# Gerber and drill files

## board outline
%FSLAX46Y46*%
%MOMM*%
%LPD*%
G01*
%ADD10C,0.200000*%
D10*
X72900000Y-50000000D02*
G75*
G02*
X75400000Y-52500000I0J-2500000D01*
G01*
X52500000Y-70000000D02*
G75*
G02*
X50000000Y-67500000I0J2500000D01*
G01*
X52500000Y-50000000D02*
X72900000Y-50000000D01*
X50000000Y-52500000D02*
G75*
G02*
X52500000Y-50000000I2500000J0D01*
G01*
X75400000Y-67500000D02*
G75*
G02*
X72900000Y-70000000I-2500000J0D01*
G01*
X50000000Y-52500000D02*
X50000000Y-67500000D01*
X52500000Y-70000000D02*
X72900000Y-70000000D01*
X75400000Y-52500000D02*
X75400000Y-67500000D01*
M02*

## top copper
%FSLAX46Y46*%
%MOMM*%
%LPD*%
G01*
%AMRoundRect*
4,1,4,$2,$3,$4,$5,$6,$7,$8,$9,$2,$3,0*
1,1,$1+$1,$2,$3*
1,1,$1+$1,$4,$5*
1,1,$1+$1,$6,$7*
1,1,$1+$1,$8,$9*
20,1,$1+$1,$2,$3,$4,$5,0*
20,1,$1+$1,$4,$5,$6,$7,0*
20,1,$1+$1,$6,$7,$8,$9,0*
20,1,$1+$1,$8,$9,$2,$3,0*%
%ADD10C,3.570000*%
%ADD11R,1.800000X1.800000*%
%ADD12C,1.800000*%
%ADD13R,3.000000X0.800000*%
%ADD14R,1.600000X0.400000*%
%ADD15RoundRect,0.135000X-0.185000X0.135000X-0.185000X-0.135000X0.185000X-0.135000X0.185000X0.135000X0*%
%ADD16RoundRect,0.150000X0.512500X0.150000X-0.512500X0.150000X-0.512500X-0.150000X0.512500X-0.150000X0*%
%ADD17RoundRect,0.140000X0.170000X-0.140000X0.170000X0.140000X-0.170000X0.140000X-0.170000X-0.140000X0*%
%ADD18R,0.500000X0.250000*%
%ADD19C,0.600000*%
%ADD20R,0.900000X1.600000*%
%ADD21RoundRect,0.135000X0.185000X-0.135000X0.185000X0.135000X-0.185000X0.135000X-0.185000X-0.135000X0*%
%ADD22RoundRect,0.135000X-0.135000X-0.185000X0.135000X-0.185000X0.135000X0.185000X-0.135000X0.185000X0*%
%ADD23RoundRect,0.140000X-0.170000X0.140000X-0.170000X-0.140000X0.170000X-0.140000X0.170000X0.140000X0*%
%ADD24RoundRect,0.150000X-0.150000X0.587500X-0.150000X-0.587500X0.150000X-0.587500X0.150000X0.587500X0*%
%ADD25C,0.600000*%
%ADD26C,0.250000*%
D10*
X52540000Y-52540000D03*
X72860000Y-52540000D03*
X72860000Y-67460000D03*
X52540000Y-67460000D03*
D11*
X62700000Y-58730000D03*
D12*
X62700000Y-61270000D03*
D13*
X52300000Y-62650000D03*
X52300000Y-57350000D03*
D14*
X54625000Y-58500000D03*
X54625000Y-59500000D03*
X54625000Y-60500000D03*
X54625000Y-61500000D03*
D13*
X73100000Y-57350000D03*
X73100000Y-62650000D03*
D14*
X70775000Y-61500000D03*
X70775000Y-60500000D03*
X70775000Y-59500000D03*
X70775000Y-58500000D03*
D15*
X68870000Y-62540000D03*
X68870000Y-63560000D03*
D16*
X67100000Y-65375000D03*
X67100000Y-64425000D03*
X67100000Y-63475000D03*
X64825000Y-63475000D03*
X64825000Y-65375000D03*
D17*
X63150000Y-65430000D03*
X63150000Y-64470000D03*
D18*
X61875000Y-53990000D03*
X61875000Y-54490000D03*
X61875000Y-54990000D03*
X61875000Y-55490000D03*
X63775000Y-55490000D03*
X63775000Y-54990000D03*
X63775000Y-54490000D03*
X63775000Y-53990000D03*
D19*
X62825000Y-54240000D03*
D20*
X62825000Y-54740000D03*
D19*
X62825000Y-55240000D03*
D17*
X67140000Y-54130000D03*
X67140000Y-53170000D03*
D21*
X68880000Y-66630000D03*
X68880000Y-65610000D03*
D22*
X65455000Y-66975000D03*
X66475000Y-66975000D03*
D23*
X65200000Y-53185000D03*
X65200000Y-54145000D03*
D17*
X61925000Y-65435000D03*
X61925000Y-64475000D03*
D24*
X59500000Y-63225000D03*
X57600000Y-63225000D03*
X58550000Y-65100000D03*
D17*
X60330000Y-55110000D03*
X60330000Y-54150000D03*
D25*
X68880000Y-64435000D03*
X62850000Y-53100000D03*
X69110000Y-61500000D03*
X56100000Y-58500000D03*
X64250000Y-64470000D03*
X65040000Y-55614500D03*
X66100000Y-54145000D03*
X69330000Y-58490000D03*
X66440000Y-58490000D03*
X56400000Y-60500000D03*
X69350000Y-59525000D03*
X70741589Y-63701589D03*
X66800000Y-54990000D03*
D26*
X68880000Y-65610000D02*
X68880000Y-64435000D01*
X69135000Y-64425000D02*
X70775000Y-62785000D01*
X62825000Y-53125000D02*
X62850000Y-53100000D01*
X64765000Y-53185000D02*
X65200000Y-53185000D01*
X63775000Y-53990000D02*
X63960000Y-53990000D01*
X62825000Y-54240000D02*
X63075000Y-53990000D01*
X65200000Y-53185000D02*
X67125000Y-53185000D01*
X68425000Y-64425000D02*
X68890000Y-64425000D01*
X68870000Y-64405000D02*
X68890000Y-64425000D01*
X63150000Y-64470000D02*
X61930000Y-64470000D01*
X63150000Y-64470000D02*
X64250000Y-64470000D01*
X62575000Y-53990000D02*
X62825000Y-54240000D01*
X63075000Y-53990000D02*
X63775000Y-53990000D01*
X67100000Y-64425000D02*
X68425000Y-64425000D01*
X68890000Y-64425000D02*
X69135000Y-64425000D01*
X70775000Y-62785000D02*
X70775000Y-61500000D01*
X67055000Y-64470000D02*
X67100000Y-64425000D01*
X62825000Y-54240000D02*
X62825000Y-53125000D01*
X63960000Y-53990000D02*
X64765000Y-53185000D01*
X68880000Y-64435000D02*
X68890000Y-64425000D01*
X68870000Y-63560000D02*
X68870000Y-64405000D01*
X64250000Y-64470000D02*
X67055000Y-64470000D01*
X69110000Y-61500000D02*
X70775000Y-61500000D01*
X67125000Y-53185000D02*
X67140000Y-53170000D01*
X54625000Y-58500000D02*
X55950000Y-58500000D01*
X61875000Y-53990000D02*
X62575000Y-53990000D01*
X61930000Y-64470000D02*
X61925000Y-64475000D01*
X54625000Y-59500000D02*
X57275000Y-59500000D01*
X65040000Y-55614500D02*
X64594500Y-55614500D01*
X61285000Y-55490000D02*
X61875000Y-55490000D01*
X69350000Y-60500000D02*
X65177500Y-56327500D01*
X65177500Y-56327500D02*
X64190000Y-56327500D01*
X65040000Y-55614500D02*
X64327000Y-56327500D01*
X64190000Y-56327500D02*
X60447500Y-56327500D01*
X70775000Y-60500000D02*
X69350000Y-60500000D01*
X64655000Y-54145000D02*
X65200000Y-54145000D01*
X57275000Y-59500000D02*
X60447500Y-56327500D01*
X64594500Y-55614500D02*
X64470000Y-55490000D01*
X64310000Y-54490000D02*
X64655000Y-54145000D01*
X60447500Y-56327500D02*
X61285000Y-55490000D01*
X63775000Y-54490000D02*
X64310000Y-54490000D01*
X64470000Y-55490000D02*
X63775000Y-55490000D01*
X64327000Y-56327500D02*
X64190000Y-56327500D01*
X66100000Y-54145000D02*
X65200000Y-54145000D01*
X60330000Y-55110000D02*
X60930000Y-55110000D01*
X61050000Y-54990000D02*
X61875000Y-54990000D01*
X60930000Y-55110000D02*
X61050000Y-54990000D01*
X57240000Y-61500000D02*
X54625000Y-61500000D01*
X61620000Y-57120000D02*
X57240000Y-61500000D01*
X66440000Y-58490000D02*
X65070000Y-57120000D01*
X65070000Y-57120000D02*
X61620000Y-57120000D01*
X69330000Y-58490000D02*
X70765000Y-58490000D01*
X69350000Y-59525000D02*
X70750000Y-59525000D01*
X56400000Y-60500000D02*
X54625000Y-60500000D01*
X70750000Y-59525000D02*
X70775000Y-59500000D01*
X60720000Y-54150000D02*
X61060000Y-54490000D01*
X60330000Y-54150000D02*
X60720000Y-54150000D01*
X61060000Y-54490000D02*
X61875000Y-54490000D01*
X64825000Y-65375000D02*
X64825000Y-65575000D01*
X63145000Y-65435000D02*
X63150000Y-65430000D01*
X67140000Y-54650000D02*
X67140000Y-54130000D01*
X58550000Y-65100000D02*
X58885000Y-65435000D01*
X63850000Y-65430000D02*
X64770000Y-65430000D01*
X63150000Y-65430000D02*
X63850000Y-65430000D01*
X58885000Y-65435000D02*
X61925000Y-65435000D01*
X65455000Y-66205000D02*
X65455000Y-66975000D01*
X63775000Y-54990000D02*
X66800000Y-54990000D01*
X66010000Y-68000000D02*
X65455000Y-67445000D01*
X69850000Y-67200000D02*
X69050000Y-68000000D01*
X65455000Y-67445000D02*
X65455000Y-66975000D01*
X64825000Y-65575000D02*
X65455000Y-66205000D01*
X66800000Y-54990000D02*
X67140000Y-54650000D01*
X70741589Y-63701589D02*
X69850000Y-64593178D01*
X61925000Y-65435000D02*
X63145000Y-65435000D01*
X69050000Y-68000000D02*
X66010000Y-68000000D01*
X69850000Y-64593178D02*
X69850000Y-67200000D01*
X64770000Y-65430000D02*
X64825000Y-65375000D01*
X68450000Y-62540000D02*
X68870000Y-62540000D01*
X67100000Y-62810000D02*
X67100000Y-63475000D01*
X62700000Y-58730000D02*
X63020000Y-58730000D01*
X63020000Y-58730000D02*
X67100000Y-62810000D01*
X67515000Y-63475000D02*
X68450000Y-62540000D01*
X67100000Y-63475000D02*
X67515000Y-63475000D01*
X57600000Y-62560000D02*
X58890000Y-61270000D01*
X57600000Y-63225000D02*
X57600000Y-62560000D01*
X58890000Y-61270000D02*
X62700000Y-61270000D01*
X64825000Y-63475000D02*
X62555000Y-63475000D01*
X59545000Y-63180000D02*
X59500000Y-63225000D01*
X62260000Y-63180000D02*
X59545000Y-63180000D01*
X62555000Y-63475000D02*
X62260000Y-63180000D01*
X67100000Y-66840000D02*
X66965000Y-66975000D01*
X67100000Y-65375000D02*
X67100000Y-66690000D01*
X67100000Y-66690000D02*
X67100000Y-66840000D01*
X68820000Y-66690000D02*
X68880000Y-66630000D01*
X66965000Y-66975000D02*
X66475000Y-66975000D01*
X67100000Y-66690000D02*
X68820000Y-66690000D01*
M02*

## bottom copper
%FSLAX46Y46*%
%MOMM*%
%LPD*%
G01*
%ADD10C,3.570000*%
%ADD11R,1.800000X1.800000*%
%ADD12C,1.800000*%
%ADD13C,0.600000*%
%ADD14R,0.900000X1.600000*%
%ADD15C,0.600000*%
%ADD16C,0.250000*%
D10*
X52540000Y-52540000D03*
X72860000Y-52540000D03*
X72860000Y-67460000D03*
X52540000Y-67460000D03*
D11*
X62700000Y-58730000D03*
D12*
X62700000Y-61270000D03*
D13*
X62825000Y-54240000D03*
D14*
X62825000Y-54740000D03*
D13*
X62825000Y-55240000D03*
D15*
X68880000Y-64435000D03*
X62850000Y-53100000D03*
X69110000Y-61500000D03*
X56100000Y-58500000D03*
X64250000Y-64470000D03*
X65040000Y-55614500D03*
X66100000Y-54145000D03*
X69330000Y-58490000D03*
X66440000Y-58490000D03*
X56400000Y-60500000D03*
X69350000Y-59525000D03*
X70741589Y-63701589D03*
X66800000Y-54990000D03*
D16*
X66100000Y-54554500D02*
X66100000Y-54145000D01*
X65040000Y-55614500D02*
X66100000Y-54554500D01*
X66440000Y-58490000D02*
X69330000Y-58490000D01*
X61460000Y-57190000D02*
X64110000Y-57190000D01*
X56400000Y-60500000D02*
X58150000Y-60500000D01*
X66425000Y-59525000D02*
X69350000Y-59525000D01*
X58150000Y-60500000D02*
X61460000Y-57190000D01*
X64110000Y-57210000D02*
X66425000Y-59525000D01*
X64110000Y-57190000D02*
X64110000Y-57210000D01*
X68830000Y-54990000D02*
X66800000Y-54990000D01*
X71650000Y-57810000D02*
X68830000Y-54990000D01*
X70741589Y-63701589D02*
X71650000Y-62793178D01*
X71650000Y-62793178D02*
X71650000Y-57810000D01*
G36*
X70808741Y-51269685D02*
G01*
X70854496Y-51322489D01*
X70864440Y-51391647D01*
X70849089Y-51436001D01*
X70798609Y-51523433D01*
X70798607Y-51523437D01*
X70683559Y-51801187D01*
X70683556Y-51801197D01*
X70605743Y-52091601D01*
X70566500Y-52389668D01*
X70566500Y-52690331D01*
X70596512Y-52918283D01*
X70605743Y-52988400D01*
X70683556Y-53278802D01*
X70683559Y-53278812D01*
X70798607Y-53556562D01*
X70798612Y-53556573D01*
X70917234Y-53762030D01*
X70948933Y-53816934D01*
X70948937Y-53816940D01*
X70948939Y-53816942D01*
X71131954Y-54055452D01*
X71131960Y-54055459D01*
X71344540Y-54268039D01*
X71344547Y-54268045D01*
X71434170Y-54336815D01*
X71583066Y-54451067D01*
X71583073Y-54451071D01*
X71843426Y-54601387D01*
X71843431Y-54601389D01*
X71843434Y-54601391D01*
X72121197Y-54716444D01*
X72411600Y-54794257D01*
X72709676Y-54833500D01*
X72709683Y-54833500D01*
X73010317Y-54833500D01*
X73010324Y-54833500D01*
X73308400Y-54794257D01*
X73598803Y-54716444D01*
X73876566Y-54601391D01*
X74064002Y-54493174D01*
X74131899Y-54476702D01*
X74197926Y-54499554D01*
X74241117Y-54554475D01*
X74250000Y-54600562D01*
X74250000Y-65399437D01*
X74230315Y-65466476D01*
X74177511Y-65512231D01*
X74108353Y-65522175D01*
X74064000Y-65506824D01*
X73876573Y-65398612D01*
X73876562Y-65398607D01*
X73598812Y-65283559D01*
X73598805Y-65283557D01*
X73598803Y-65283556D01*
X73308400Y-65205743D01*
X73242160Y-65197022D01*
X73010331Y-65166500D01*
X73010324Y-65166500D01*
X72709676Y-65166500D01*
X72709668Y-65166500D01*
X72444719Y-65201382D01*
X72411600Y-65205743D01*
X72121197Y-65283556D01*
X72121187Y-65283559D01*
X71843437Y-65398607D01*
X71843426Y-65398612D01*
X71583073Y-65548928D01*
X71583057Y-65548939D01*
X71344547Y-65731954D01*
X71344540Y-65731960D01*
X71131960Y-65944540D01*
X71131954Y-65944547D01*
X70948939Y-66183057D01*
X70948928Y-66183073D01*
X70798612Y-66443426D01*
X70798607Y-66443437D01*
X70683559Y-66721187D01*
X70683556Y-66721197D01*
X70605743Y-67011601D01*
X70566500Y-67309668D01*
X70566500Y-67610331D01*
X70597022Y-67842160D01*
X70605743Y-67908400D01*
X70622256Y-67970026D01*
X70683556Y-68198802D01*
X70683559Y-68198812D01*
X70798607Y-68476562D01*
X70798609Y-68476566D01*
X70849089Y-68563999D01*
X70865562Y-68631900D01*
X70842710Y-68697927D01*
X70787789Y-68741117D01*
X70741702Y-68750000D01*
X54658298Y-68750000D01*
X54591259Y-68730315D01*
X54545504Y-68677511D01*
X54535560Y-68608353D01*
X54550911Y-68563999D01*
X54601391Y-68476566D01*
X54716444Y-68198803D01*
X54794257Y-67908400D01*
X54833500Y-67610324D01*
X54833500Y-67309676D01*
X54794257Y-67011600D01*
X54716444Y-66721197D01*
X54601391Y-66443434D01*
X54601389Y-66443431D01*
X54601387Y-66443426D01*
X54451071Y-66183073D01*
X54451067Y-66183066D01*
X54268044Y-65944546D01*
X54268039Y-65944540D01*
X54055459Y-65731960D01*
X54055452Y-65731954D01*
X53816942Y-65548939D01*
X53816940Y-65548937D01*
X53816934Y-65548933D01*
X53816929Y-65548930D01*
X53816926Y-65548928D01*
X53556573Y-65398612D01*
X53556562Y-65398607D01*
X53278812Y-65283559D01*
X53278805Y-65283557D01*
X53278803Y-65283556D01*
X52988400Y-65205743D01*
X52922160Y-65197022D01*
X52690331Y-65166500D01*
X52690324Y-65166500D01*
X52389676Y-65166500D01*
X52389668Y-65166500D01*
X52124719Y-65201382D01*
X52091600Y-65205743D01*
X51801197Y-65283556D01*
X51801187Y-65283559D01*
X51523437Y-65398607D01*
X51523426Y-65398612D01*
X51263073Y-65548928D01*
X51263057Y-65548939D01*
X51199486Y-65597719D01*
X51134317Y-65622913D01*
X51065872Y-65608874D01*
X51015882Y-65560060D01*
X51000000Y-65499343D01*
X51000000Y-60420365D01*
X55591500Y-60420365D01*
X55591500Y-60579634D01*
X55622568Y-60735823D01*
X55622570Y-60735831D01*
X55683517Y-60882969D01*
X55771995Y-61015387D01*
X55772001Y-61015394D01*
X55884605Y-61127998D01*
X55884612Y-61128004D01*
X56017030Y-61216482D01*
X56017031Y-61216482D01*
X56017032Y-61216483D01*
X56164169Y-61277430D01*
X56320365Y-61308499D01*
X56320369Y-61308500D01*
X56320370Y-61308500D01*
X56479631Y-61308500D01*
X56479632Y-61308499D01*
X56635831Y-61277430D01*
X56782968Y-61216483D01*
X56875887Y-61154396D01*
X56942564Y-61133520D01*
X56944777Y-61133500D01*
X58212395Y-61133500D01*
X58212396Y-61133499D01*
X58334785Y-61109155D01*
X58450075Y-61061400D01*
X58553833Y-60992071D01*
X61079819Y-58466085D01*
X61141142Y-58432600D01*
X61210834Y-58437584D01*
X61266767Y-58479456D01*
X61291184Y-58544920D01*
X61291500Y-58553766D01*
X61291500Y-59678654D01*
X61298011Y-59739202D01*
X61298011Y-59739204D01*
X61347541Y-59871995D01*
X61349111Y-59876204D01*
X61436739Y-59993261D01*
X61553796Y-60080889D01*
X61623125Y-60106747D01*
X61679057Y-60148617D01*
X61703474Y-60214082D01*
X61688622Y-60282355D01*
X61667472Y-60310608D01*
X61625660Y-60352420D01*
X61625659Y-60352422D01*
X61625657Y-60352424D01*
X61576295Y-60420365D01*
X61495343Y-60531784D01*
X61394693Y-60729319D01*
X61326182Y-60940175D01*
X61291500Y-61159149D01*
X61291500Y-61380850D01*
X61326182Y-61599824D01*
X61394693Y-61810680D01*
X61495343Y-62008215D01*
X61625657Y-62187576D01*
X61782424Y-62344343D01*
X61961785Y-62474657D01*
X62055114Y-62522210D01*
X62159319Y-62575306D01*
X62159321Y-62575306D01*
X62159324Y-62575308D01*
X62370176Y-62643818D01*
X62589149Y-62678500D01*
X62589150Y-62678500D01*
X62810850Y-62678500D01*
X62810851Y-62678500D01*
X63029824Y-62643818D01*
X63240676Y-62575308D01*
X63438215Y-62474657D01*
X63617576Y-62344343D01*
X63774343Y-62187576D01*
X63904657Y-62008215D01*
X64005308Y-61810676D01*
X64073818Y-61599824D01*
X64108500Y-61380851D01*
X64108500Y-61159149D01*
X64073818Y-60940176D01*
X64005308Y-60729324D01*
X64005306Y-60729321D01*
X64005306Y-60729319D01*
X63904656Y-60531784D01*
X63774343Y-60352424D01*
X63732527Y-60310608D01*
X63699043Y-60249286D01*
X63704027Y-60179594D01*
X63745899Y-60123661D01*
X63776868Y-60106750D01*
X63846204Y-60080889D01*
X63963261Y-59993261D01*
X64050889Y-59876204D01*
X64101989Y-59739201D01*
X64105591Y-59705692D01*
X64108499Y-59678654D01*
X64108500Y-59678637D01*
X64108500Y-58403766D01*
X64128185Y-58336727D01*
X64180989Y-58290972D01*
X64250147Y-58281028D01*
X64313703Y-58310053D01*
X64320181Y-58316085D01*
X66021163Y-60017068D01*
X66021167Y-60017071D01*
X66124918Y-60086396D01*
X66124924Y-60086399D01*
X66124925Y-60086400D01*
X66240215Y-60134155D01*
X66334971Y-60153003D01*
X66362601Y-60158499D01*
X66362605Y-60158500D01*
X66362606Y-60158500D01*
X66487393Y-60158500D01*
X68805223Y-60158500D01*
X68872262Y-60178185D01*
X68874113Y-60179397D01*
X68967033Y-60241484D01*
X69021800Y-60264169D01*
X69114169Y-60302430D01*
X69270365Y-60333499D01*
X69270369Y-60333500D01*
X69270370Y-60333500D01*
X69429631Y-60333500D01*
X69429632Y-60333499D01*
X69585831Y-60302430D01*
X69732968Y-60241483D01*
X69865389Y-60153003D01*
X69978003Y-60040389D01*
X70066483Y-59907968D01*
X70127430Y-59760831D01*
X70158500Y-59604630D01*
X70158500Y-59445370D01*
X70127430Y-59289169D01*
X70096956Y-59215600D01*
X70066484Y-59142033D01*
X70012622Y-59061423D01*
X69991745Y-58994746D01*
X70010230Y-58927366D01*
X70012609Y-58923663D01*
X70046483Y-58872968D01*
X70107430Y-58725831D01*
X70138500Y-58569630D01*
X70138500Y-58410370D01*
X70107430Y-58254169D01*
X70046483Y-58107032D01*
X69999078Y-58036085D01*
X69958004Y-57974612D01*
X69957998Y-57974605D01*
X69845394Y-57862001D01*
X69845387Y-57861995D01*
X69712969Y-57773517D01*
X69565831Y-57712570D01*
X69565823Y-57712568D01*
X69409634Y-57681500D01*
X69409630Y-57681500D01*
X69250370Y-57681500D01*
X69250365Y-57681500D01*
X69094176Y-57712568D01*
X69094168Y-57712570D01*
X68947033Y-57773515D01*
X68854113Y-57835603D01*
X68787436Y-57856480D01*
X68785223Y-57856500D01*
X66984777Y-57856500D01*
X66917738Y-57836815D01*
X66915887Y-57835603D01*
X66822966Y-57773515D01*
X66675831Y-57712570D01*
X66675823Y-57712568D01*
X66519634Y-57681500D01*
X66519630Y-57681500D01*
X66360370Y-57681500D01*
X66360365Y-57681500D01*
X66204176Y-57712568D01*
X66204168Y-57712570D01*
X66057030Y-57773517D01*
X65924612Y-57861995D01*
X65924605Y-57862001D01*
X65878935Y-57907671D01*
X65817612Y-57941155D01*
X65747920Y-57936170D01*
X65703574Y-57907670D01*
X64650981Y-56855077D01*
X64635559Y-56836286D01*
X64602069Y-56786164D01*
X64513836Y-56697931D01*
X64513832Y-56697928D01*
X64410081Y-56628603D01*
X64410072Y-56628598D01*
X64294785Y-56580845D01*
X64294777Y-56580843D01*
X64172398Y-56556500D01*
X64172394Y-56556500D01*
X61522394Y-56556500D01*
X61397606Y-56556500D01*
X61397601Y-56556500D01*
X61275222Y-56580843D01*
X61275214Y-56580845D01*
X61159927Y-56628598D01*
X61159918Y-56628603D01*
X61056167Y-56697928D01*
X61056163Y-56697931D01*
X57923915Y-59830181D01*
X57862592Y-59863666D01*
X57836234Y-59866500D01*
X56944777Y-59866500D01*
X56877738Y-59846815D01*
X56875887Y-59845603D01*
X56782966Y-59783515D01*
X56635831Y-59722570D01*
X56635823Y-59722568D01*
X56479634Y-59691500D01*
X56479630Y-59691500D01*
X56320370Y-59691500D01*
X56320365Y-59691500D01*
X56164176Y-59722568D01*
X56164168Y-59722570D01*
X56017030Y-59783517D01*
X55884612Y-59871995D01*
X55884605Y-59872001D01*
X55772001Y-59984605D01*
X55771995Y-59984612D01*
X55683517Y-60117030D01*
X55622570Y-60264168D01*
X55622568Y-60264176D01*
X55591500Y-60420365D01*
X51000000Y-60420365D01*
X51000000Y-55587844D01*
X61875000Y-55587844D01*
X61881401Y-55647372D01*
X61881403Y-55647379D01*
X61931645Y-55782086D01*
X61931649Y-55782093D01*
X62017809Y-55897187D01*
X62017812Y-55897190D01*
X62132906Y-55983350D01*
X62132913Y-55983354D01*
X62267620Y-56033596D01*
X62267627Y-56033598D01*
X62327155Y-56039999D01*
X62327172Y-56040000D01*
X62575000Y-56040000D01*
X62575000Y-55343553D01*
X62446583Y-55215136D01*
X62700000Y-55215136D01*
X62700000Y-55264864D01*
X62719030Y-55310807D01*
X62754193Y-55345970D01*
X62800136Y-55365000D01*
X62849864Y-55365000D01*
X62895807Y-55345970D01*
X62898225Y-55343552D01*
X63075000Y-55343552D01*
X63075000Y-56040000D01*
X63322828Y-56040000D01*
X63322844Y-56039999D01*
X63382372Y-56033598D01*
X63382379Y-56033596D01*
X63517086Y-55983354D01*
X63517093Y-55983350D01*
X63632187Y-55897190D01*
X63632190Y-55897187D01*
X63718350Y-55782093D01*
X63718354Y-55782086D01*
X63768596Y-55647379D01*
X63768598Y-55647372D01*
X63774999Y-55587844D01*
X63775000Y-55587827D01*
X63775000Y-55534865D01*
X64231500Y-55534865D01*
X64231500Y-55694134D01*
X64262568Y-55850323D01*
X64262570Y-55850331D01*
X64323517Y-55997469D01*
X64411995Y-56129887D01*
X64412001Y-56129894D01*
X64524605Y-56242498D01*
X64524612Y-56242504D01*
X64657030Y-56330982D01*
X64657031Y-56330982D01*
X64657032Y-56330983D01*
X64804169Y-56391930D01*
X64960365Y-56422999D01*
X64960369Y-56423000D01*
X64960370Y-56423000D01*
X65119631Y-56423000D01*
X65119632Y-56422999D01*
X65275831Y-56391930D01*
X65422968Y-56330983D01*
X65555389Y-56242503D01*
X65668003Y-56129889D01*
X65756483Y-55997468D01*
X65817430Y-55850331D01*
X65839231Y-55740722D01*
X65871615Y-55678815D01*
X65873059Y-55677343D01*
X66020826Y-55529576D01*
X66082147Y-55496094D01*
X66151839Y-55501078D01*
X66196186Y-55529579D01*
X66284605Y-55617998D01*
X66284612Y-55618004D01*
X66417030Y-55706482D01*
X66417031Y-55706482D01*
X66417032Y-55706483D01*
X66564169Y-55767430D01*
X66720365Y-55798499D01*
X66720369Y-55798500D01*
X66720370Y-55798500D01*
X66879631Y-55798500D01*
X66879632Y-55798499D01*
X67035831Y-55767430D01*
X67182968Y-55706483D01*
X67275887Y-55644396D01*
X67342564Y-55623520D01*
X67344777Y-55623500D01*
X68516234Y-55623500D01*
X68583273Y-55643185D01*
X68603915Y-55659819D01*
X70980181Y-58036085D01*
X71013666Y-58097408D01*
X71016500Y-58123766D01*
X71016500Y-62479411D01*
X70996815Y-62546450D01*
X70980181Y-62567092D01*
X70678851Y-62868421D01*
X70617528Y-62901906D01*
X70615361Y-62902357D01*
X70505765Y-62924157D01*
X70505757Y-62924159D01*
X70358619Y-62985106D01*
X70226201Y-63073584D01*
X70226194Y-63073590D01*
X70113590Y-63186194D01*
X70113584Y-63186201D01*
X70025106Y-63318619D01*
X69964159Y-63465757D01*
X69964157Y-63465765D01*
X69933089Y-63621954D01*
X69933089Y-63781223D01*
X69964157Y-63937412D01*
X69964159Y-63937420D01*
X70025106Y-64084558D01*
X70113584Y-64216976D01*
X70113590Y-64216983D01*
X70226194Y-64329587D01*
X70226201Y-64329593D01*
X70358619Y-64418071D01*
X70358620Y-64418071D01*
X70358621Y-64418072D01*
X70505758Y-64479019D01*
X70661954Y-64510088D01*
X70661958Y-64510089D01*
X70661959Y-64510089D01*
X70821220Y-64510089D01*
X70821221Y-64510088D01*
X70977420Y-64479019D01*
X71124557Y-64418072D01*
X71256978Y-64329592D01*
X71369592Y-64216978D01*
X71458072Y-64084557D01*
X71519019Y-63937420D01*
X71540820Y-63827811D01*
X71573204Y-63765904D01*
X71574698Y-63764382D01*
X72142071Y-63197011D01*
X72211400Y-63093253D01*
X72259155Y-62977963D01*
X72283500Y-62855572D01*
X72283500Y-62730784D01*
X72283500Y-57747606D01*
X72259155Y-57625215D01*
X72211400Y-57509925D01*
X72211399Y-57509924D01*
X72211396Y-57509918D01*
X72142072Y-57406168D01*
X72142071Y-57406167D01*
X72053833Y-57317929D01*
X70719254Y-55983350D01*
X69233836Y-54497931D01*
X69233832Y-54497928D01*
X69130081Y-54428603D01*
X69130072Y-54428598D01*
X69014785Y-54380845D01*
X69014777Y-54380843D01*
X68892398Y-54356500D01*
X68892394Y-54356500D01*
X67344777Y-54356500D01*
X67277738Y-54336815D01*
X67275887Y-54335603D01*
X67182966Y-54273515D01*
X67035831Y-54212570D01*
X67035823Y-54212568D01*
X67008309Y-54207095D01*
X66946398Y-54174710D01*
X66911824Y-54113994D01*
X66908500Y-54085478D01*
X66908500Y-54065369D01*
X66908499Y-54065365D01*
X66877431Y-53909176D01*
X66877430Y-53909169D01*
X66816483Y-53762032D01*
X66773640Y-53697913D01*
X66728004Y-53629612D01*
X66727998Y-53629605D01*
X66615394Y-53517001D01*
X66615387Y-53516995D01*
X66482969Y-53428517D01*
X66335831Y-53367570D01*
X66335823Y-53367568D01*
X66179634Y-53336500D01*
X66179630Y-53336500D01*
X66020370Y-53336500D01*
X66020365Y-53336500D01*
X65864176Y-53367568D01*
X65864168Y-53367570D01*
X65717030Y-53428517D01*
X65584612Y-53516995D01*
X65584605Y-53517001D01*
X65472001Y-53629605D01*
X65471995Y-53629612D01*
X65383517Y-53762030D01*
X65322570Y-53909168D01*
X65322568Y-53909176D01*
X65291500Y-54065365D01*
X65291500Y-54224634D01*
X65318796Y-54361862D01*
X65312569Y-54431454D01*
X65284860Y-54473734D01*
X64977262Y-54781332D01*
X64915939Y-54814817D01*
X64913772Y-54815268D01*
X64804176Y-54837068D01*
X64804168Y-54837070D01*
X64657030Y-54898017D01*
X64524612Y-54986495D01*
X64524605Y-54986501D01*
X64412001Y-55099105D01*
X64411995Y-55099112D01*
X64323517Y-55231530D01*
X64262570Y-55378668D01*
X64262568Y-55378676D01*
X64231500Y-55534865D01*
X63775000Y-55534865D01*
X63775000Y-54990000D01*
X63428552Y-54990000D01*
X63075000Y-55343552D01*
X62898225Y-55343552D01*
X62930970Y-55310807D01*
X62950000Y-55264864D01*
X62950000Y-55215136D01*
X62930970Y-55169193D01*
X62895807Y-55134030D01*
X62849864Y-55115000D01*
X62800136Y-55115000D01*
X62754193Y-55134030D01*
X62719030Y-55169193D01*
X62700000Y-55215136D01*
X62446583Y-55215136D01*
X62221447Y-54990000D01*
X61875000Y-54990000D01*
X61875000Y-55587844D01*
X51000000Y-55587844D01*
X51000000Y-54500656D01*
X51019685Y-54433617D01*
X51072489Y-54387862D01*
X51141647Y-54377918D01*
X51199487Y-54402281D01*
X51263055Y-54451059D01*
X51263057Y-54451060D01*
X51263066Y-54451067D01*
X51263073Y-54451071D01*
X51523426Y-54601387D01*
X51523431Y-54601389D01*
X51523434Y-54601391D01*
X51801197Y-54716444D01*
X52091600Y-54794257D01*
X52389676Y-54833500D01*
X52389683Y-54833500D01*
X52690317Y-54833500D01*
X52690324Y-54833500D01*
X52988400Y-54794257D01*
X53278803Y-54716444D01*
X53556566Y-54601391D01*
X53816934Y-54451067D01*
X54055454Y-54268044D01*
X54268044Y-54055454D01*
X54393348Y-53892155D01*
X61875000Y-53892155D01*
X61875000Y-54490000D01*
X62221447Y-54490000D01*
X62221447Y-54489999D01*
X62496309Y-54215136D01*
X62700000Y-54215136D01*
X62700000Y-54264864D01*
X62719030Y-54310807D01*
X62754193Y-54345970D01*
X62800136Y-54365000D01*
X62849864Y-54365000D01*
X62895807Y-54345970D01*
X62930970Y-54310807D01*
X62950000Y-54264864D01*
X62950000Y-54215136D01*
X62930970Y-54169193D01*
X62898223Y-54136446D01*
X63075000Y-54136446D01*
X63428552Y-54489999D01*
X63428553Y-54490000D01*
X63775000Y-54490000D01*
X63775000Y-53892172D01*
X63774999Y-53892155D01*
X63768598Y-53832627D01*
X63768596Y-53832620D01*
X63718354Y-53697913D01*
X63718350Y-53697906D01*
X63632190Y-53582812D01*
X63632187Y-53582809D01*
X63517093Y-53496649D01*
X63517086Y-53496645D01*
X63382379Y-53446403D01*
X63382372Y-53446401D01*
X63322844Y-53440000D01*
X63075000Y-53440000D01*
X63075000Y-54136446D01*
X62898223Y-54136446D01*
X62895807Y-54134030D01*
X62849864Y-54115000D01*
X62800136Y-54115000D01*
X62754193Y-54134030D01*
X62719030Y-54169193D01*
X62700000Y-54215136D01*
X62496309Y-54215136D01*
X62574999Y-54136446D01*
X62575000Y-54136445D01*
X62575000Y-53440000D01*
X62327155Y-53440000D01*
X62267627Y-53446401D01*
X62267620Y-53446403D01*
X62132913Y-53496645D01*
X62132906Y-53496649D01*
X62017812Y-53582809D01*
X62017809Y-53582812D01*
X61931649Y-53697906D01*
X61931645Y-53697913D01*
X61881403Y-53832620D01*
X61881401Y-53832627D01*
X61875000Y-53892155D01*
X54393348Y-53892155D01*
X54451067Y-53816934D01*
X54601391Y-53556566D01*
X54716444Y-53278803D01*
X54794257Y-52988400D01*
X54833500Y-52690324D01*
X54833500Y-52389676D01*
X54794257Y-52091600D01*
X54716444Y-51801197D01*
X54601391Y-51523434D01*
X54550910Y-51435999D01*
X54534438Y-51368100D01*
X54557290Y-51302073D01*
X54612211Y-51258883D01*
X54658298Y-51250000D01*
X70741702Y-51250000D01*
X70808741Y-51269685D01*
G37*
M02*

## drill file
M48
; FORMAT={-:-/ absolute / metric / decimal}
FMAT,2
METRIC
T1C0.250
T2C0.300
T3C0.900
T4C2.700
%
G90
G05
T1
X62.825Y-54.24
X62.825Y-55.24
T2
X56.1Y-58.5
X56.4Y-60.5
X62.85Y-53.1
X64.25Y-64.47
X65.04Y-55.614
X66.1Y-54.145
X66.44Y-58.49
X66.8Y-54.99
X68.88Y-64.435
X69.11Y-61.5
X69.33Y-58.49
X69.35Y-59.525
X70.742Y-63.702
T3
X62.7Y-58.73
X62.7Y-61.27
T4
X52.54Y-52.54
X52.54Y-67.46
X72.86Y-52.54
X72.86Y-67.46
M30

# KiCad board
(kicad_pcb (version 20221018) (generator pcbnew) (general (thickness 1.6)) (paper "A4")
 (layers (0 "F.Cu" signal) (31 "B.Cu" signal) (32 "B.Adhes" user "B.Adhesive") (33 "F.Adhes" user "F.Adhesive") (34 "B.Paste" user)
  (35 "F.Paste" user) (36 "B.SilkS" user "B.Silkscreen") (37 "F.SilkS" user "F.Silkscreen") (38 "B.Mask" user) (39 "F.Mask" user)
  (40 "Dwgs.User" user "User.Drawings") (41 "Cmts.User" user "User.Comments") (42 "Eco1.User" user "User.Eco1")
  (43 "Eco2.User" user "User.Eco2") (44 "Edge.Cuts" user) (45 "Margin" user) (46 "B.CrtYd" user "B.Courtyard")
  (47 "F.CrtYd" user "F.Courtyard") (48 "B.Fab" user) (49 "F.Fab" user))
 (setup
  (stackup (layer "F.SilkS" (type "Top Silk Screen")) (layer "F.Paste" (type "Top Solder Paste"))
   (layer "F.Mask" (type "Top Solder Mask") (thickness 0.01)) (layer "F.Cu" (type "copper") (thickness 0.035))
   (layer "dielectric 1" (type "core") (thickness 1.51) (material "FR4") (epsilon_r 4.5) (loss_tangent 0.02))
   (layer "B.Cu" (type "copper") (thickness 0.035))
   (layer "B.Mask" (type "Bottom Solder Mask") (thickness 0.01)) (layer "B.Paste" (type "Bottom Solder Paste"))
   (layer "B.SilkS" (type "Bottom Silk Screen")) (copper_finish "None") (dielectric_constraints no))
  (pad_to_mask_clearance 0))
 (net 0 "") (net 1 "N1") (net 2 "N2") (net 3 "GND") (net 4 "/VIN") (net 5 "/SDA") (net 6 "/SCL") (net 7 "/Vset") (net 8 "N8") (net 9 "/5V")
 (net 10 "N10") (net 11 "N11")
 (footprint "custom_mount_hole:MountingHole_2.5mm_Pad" (layer "F.Cu") (at 52.54 52.54)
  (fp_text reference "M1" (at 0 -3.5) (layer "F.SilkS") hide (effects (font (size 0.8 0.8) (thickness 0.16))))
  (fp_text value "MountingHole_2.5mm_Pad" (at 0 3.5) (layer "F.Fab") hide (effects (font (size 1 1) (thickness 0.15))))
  (pad "~" thru_hole circle (at 0 0) (size 3.57 3.57) (drill 2.7) (layers "*.Cu" "*.Mask")))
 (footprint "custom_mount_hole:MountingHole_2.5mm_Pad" (layer "F.Cu") (at 72.86 52.54)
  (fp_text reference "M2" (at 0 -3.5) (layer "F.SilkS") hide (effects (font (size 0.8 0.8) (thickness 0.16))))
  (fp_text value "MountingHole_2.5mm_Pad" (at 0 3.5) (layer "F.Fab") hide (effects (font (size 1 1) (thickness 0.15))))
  (pad "~" thru_hole circle (at 0 0) (size 3.57 3.57) (drill 2.7) (layers "*.Cu" "*.Mask")))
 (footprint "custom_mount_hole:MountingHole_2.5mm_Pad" (layer "F.Cu") (at 72.86 67.46)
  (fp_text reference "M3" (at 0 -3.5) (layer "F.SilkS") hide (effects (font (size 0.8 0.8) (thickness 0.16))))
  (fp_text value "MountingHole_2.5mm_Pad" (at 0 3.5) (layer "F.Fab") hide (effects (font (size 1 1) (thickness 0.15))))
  (pad "~" thru_hole circle (at 0 0) (size 3.57 3.57) (drill 2.7) (layers "*.Cu" "*.Mask")))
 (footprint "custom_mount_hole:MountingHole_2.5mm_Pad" (layer "F.Cu") (at 52.54 67.46)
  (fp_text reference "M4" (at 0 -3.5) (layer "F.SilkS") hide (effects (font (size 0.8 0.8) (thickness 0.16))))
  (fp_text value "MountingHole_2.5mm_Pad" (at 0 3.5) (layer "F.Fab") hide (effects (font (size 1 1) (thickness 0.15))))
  (pad "~" thru_hole circle (at 0 0) (size 3.57 3.57) (drill 2.7) (layers "*.Cu" "*.Mask")))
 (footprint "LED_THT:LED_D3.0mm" (layer "F.Cu") (at 62.7 58.73 -90)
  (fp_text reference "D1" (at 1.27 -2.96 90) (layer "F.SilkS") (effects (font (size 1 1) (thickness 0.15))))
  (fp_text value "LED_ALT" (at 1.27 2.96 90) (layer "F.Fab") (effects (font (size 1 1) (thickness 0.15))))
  (pad "1" thru_hole rect (at 0 0 270) (size 1.8 1.8) (drill 0.9) (layers "*.Cu" "*.Mask") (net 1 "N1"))
  (pad "2" thru_hole circle (at 2.54 0 270) (size 1.8 1.8) (drill 0.9) (layers "*.Cu" "*.Mask") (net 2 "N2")))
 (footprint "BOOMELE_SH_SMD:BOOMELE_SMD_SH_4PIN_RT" (layer "F.Cu") (at 52.78 60 90)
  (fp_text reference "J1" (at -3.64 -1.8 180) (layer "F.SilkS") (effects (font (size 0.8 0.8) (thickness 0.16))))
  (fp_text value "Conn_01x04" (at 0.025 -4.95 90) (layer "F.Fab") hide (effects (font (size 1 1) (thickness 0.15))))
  (pad "" smd rect (at -2.65 -0.48 270) (size 0.8 3) (layers "F.Cu" "F.Paste" "F.Mask"))
  (pad "" smd rect (at 2.65 -0.48 270) (size 0.8 3) (layers "F.Cu" "F.Paste" "F.Mask"))
  (pad "1" smd rect (at 1.5 1.845 270) (size 0.4 1.6) (layers "F.Cu" "F.Paste" "F.Mask") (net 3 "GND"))
  (pad "2" smd rect (at 0.5 1.845 270) (size 0.4 1.6) (layers "F.Cu" "F.Paste" "F.Mask") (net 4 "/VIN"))
  (pad "3" smd rect (at -0.5 1.845 270) (size 0.4 1.6) (layers "F.Cu" "F.Paste" "F.Mask") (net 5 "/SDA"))
  (pad "4" smd rect (at -1.5 1.845 270) (size 0.4 1.6) (layers "F.Cu" "F.Paste" "F.Mask") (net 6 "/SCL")))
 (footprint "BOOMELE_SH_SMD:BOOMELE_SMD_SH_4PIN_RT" (layer "F.Cu") (at 72.62 60 -90)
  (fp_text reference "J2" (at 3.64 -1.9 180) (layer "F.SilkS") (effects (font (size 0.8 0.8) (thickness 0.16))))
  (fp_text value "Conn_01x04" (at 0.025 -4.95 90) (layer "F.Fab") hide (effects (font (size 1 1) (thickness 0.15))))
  (pad "" smd rect (at -2.65 -0.48 90) (size 0.8 3) (layers "F.Cu" "F.Paste" "F.Mask"))
  (pad "" smd rect (at 2.65 -0.48 90) (size 0.8 3) (layers "F.Cu" "F.Paste" "F.Mask"))
  (pad "1" smd rect (at 1.5 1.845 90) (size 0.4 1.6) (layers "F.Cu" "F.Paste" "F.Mask") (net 3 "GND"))
  (pad "2" smd rect (at 0.5 1.845 90) (size 0.4 1.6) (layers "F.Cu" "F.Paste" "F.Mask") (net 4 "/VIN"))
  (pad "3" smd rect (at -0.5 1.845 90) (size 0.4 1.6) (layers "F.Cu" "F.Paste" "F.Mask") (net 5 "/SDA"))
  (pad "4" smd rect (at -1.5 1.845 90) (size 0.4 1.6) (layers "F.Cu" "F.Paste" "F.Mask") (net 6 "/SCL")))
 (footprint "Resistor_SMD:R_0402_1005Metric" (layer "F.Cu") (at 68.87 63.05 -90)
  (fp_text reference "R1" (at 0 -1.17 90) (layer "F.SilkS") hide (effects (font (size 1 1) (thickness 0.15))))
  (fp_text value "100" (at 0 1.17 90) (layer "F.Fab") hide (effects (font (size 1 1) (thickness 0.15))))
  (pad "1" smd roundrect (at -0.51 0 270) (size 0.54 0.64) (layers "F.Cu" "F.Paste" "F.Mask") (roundrect_rratio 0.25) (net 1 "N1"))
  (pad "2" smd roundrect (at 0.51 0 270) (size 0.54 0.64) (layers "F.Cu" "F.Paste" "F.Mask") (roundrect_rratio 0.25) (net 3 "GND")))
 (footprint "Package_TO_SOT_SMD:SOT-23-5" (layer "F.Cu") (at 65.9625 64.425 180)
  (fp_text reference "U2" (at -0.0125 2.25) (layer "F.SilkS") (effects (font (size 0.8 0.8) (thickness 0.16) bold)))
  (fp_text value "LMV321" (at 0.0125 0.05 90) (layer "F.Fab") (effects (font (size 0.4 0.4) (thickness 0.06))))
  (pad "1" smd roundrect (at -1.1375 -0.95 180) (size 1.325 0.6) (layers "F.Cu" "F.Paste" "F.Mask") (roundrect_rratio 0.25) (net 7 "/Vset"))
  (pad "2" smd roundrect (at -1.1375 0 180) (size 1.325 0.6) (layers "F.Cu" "F.Paste" "F.Mask") (roundrect_rratio 0.25) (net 3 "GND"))
  (pad "3" smd roundrect (at -1.1375 0.95 180) (size 1.325 0.6) (layers "F.Cu" "F.Paste" "F.Mask") (roundrect_rratio 0.25) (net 1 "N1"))
  (pad "4" smd roundrect (at 1.1375 0.95 180) (size 1.325 0.6) (layers "F.Cu" "F.Paste" "F.Mask") (roundrect_rratio 0.25) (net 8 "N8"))
  (pad "5" smd roundrect (at 1.1375 -0.95 180) (size 1.325 0.6) (layers "F.Cu" "F.Paste" "F.Mask") (roundrect_rratio 0.25) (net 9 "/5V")))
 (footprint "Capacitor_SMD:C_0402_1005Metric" (layer "F.Cu") (at 63.15 64.95 90)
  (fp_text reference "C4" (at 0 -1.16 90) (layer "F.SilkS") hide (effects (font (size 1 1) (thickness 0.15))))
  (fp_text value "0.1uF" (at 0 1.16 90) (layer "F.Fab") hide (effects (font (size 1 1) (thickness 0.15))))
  (pad "1" smd roundrect (at -0.48 0 90) (size 0.56 0.62) (layers "F.Cu" "F.Paste" "F.Mask") (roundrect_rratio 0.25) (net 9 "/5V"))
  (pad "2" smd roundrect (at 0.48 0 90) (size 0.56 0.62) (layers "F.Cu" "F.Paste" "F.Mask") (roundrect_rratio 0.25) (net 3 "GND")))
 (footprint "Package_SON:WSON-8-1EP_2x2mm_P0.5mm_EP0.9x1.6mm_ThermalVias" (layer "F.Cu") (at 62.825 54.74)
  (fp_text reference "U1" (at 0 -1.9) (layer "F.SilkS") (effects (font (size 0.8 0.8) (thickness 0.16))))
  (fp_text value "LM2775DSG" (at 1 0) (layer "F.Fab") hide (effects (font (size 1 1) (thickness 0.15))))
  (pad "" smd rect (at 0 -0.4) (size 0.75 0.65) (layers "F.Paste"))
  (pad "" smd rect (at 0 0.4) (size 0.75 0.65) (layers "F.Paste"))
  (pad "1" smd rect (at -0.95 -0.75) (size 0.5 0.25) (layers "F.Cu" "F.Paste" "F.Mask") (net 3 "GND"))
  (pad "2" smd rect (at -0.95 -0.25) (size 0.5 0.25) (layers "F.Cu" "F.Paste" "F.Mask") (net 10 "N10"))
  (pad "3" smd rect (at -0.95 0.25) (size 0.5 0.25) (layers "F.Cu" "F.Paste" "F.Mask") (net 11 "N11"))
  (pad "4" smd rect (at -0.95 0.75) (size 0.5 0.25) (layers "F.Cu" "F.Paste" "F.Mask") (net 4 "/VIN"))
  (pad "5" smd rect (at 0.95 0.75) (size 0.5 0.25) (layers "F.Cu" "F.Paste" "F.Mask") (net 4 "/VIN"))
  (pad "6" smd rect (at 0.95 0.25) (size 0.5 0.25) (layers "F.Cu" "F.Paste" "F.Mask") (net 9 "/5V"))
  (pad "7" smd rect (at 0.95 -0.25) (size 0.5 0.25) (layers "F.Cu" "F.Paste" "F.Mask") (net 4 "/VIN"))
  (pad "8" smd rect (at 0.95 -0.75) (size 0.5 0.25) (layers "F.Cu" "F.Paste" "F.Mask") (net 3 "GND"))
  (pad "9" thru_hole circle (at 0 -0.5) (size 0.6 0.6) (drill 0.25) (layers "*.Cu") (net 3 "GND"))
  (pad "9" smd rect (at 0 0) (size 0.9 1.6) (layers "F.Cu" "F.Mask") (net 3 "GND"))
  (pad "9" smd rect (at 0 0) (size 0.9 1.6) (layers "B.Cu") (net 3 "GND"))
  (pad "9" thru_hole circle (at 0 0.5) (size 0.6 0.6) (drill 0.25) (layers "*.Cu") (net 3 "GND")))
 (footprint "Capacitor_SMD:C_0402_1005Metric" (layer "F.Cu") (at 67.14 53.65 90)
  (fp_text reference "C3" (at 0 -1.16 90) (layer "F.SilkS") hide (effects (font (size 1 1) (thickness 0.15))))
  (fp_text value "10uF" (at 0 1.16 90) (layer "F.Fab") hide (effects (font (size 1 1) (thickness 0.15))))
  (pad "1" smd roundrect (at -0.48 0 90) (size 0.56 0.62) (layers "F.Cu" "F.Paste" "F.Mask") (roundrect_rratio 0.25) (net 9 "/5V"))
  (pad "2" smd roundrect (at 0.48 0 90) (size 0.56 0.62) (layers "F.Cu" "F.Paste" "F.Mask") (roundrect_rratio 0.25) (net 3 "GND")))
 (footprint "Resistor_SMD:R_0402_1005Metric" (layer "F.Cu") (at 68.88 66.12 90)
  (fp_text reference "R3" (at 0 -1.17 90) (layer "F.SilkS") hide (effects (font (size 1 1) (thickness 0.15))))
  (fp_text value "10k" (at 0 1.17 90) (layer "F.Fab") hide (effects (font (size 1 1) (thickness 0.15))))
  (pad "1" smd roundrect (at -0.51 0 90) (size 0.54 0.64) (layers "F.Cu" "F.Paste" "F.Mask") (roundrect_rratio 0.25) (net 7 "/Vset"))
  (pad "2" smd roundrect (at 0.51 0 90) (size 0.54 0.64) (layers "F.Cu" "F.Paste" "F.Mask") (roundrect_rratio 0.25) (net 3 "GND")))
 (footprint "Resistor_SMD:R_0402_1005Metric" (layer "F.Cu") (at 65.965 66.975)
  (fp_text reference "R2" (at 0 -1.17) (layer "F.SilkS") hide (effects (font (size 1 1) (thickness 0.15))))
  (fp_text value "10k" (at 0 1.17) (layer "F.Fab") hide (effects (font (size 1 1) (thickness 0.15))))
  (pad "1" smd roundrect (at -0.51 0) (size 0.54 0.64) (layers "F.Cu" "F.Paste" "F.Mask") (roundrect_rratio 0.25) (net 9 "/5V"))
  (pad "2" smd roundrect (at 0.51 0) (size 0.54 0.64) (layers "F.Cu" "F.Paste" "F.Mask") (roundrect_rratio 0.25) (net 7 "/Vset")))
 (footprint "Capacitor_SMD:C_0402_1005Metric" (layer "F.Cu") (at 65.2 53.665 -90)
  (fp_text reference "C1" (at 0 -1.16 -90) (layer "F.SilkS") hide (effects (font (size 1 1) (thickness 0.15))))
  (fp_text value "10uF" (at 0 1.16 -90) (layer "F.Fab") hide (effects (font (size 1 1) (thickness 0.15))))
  (pad "1" smd roundrect (at -0.48 0 270) (size 0.56 0.62) (layers "F.Cu" "F.Paste" "F.Mask") (roundrect_rratio 0.25) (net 3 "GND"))
  (pad "2" smd roundrect (at 0.48 0 270) (size 0.56 0.62) (layers "F.Cu" "F.Paste" "F.Mask") (roundrect_rratio 0.25) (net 4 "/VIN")))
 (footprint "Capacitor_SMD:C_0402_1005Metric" (layer "F.Cu") (at 61.925 64.955 90)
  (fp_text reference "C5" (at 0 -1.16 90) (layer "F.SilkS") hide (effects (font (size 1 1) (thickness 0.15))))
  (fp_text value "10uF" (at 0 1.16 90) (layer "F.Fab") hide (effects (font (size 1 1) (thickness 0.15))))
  (pad "1" smd roundrect (at -0.48 0 90) (size 0.56 0.62) (layers "F.Cu" "F.Paste" "F.Mask") (roundrect_rratio 0.25) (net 9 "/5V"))
  (pad "2" smd roundrect (at 0.48 0 90) (size 0.56 0.62) (layers "F.Cu" "F.Paste" "F.Mask") (roundrect_rratio 0.25) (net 3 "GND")))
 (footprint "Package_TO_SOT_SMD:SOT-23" (layer "F.Cu") (at 58.55 64.1625 -90)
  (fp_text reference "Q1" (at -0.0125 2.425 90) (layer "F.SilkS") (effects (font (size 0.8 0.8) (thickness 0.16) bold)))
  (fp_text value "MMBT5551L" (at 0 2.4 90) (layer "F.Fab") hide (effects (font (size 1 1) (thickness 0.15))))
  (pad "1" smd roundrect (at -0.9375 -0.95 270) (size 1.475 0.6) (layers "F.Cu" "F.Paste" "F.Mask") (roundrect_rratio 0.25) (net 8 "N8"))
  (pad "2" smd roundrect (at -0.9375 0.95 270) (size 1.475 0.6) (layers "F.Cu" "F.Paste" "F.Mask") (roundrect_rratio 0.25) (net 2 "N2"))
  (pad "3" smd roundrect (at 0.9375 0 270) (size 1.475 0.6) (layers "F.Cu" "F.Paste" "F.Mask") (roundrect_rratio 0.25) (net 9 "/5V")))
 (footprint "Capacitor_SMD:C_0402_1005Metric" (layer "F.Cu") (at 60.33 54.63 90)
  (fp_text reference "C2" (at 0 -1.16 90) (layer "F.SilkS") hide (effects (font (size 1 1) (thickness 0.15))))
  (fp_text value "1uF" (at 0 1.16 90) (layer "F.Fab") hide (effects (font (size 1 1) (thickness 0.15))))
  (pad "1" smd roundrect (at -0.48 0 90) (size 0.56 0.62) (layers "F.Cu" "F.Paste" "F.Mask") (roundrect_rratio 0.25) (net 11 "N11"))
  (pad "2" smd roundrect (at 0.48 0 90) (size 0.56 0.62) (layers "F.Cu" "F.Paste" "F.Mask") (roundrect_rratio 0.25) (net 10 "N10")))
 (gr_arc (start 72.9 50) (mid 74.667767 50.732233) (end 75.4 52.5) (stroke (width 0.2) (type solid)) (layer "Edge.Cuts"))
 (gr_arc (start 52.5 70) (mid 50.732233 69.267767) (end 50 67.5) (stroke (width 0.2) (type solid)) (layer "Edge.Cuts"))
 (gr_line (start 52.5 50) (end 72.9 50) (stroke (width 0.2) (type solid)) (layer "Edge.Cuts"))
 (gr_arc (start 50 52.5) (mid 50.732233 50.732233) (end 52.5 50) (stroke (width 0.2) (type solid)) (layer "Edge.Cuts"))
 (gr_arc (start 75.4 67.5) (mid 74.667767 69.267767) (end 72.9 70) (stroke (width 0.2) (type solid)) (layer "Edge.Cuts"))
 (gr_line (start 50 52.5) (end 50 67.5) (stroke (width 0.2) (type solid)) (layer "Edge.Cuts"))
 (gr_line (start 52.5 70) (end 72.9 70) (stroke (width 0.2) (type solid)) (layer "Edge.Cuts"))
 (gr_line (start 75.4 52.5) (end 75.4 67.5) (stroke (width 0.2) (type solid)) (layer "Edge.Cuts"))
 (segment (start 68.88 65.61) (end 68.88 64.435) (width 0.25) (layer "F.Cu") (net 3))
 (segment (start 69.135 64.425) (end 70.775 62.785) (width 0.25) (layer "F.Cu") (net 3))
 (segment (start 62.825 53.125) (end 62.85 53.1) (width 0.25) (layer "F.Cu") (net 3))
 (segment (start 64.765 53.185) (end 65.2 53.185) (width 0.25) (layer "F.Cu") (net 3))
 (segment (start 63.775 53.99) (end 63.96 53.99) (width 0.25) (layer "F.Cu") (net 3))
 (segment (start 62.825 54.24) (end 63.075 53.99) (width 0.25) (layer "F.Cu") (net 3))
 (segment (start 65.2 53.185) (end 67.125 53.185) (width 0.25) (layer "F.Cu") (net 3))
 (segment (start 68.425 64.425) (end 68.89 64.425) (width 0.25) (layer "F.Cu") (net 3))
 (segment (start 68.87 64.405) (end 68.89 64.425) (width 0.25) (layer "F.Cu") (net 3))
 (segment (start 63.15 64.47) (end 61.93 64.47) (width 0.25) (layer "F.Cu") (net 3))
 (segment (start 63.15 64.47) (end 64.25 64.47) (width 0.25) (layer "F.Cu") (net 3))
 (segment (start 62.575 53.99) (end 62.825 54.24) (width 0.25) (layer "F.Cu") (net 3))
 (segment (start 63.075 53.99) (end 63.775 53.99) (width 0.25) (layer "F.Cu") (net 3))
 (segment (start 67.1 64.425) (end 68.425 64.425) (width 0.25) (layer "F.Cu") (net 3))
 (segment (start 68.89 64.425) (end 69.135 64.425) (width 0.25) (layer "F.Cu") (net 3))
 (segment (start 70.775 62.785) (end 70.775 61.5) (width 0.25) (layer "F.Cu") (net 3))
 (segment (start 67.055 64.47) (end 67.1 64.425) (width 0.25) (layer "F.Cu") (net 3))
 (segment (start 62.825 54.24) (end 62.825 53.125) (width 0.25) (layer "F.Cu") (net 3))
 (segment (start 63.96 53.99) (end 64.765 53.185) (width 0.25) (layer "F.Cu") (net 3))
 (segment (start 68.88 64.435) (end 68.89 64.425) (width 0.25) (layer "F.Cu") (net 3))
 (segment (start 68.87 63.56) (end 68.87 64.405) (width 0.25) (layer "F.Cu") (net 3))
 (segment (start 64.25 64.47) (end 67.055 64.47) (width 0.25) (layer "F.Cu") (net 3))
 (segment (start 69.11 61.5) (end 70.775 61.5) (width 0.25) (layer "F.Cu") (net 3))
 (segment (start 67.125 53.185) (end 67.14 53.17) (width 0.25) (layer "F.Cu") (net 3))
 (segment (start 54.625 58.5) (end 55.95 58.5) (width 0.25) (layer "F.Cu") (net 3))
 (segment (start 61.875 53.99) (end 62.575 53.99) (width 0.25) (layer "F.Cu") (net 3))
 (segment (start 61.93 64.47) (end 61.925 64.475) (width 0.25) (layer "F.Cu") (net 3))
 (via (at 68.88 64.435) (size 0.6) (drill 0.3) (layers "F.Cu" "B.Cu") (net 3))
 (via (at 62.85 53.1) (size 0.6) (drill 0.3) (layers "F.Cu" "B.Cu") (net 3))
 (via (at 69.11 61.5) (size 0.6) (drill 0.3) (layers "F.Cu" "B.Cu") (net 3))
 (via (at 56.1 58.5) (size 0.6) (drill 0.3) (layers "F.Cu" "B.Cu") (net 3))
 (via (at 64.25 64.47) (size 0.6) (drill 0.3) (layers "F.Cu" "B.Cu") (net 3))
 (segment (start 54.625 59.5) (end 57.275 59.5) (width 0.25) (layer "F.Cu") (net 4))
 (segment (start 65.04 55.6145) (end 64.5945 55.6145) (width 0.25) (layer "F.Cu") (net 4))
 (segment (start 61.285 55.49) (end 61.875 55.49) (width 0.25) (layer "F.Cu") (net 4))
 (segment (start 69.35 60.5) (end 65.1775 56.3275) (width 0.25) (layer "F.Cu") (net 4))
 (segment (start 65.1775 56.3275) (end 64.19 56.3275) (width 0.25) (layer "F.Cu") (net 4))
 (segment (start 65.04 55.6145) (end 64.327 56.3275) (width 0.25) (layer "F.Cu") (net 4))
 (segment (start 64.19 56.3275) (end 60.4475 56.3275) (width 0.25) (layer "F.Cu") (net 4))
 (segment (start 70.775 60.5) (end 69.35 60.5) (width 0.25) (layer "F.Cu") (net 4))
 (segment (start 64.655 54.145) (end 65.2 54.145) (width 0.25) (layer "F.Cu") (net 4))
 (segment (start 57.275 59.5) (end 60.4475 56.3275) (width 0.25) (layer "F.Cu") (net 4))
 (segment (start 64.5945 55.6145) (end 64.47 55.49) (width 0.25) (layer "F.Cu") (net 4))
 (segment (start 64.31 54.49) (end 64.655 54.145) (width 0.25) (layer "F.Cu") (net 4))
 (segment (start 60.4475 56.3275) (end 61.285 55.49) (width 0.25) (layer "F.Cu") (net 4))
 (segment (start 63.775 54.49) (end 64.31 54.49) (width 0.25) (layer "F.Cu") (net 4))
 (segment (start 64.47 55.49) (end 63.775 55.49) (width 0.25) (layer "F.Cu") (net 4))
 (segment (start 64.327 56.3275) (end 64.19 56.3275) (width 0.25) (layer "F.Cu") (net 4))
 (segment (start 66.1 54.145) (end 65.2 54.145) (width 0.25) (layer "F.Cu") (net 4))
 (via (at 65.04 55.6145) (size 0.6) (drill 0.3) (layers "F.Cu" "B.Cu") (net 4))
 (via (at 66.1 54.145) (size 0.6) (drill 0.3) (layers "F.Cu" "B.Cu") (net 4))
 (segment (start 66.1 54.5545) (end 66.1 54.145) (width 0.25) (layer "B.Cu") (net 4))
 (segment (start 65.04 55.6145) (end 66.1 54.5545) (width 0.25) (layer "B.Cu") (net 4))
 (segment (start 60.33 55.11) (end 60.93 55.11) (width 0.25) (layer "F.Cu") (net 11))
 (segment (start 61.05 54.99) (end 61.875 54.99) (width 0.25) (layer "F.Cu") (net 11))
 (segment (start 60.93 55.11) (end 61.05 54.99) (width 0.25) (layer "F.Cu") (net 11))
 (segment (start 57.24 61.5) (end 54.625 61.5) (width 0.25) (layer "F.Cu") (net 6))
 (segment (start 61.62 57.12) (end 57.24 61.5) (width 0.25) (layer "F.Cu") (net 6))
 (segment (start 66.44 58.49) (end 65.07 57.12) (width 0.25) (layer "F.Cu") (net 6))
 (segment (start 65.07 57.12) (end 61.62 57.12) (width 0.25) (layer "F.Cu") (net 6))
 (segment (start 69.33 58.49) (end 70.765 58.49) (width 0.25) (layer "F.Cu") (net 6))
 (via (at 69.33 58.49) (size 0.6) (drill 0.3) (layers "F.Cu" "B.Cu") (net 6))
 (via (at 66.44 58.49) (size 0.6) (drill 0.3) (layers "F.Cu" "B.Cu") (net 6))
 (segment (start 66.44 58.49) (end 69.33 58.49) (width 0.25) (layer "B.Cu") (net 6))
 (segment (start 69.35 59.525) (end 70.75 59.525) (width 0.25) (layer "F.Cu") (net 5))
 (segment (start 56.4 60.5) (end 54.625 60.5) (width 0.25) (layer "F.Cu") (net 5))
 (segment (start 70.75 59.525) (end 70.775 59.5) (width 0.25) (layer "F.Cu") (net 5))
 (via (at 56.4 60.5) (size 0.6) (drill 0.3) (layers "F.Cu" "B.Cu") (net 5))
 (via (at 69.35 59.525) (size 0.6) (drill 0.3) (layers "F.Cu" "B.Cu") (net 5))
 (segment (start 61.46 57.19) (end 64.11 57.19) (width 0.25) (layer "B.Cu") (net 5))
 (segment (start 56.4 60.5) (end 58.15 60.5) (width 0.25) (layer "B.Cu") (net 5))
 (segment (start 66.425 59.525) (end 69.35 59.525) (width 0.25) (layer "B.Cu") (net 5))
 (segment (start 58.15 60.5) (end 61.46 57.19) (width 0.25) (layer "B.Cu") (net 5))
 (segment (start 64.11 57.21) (end 66.425 59.525) (width 0.25) (layer "B.Cu") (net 5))
 (segment (start 64.11 57.19) (end 64.11 57.21) (width 0.25) (layer "B.Cu") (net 5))
 (segment (start 60.72 54.15) (end 61.06 54.49) (width 0.25) (layer "F.Cu") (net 10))
 (segment (start 60.33 54.15) (end 60.72 54.15) (width 0.25) (layer "F.Cu") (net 10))
 (segment (start 61.06 54.49) (end 61.875 54.49) (width 0.25) (layer "F.Cu") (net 10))
 (segment (start 64.825 65.375) (end 64.825 65.575) (width 0.25) (layer "F.Cu") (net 9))
 (segment (start 63.145 65.435) (end 63.15 65.43) (width 0.25) (layer "F.Cu") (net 9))
 (segment (start 67.14 54.65) (end 67.14 54.13) (width 0.25) (layer "F.Cu") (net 9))
 (segment (start 58.55 65.1) (end 58.885 65.435) (width 0.25) (layer "F.Cu") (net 9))
 (segment (start 63.85 65.43) (end 64.77 65.43) (width 0.25) (layer "F.Cu") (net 9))
 (segment (start 63.15 65.43) (end 63.85 65.43) (width 0.25) (layer "F.Cu") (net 9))
 (segment (start 58.885 65.435) (end 61.925 65.435) (width 0.25) (layer "F.Cu") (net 9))
 (segment (start 65.455 66.205) (end 65.455 66.975) (width 0.25) (layer "F.Cu") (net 9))
 (segment (start 63.775 54.99) (end 66.8 54.99) (width 0.25) (layer "F.Cu") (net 9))
 (segment (start 66.01 68) (end 65.455 67.445) (width 0.25) (layer "F.Cu") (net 9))
 (segment (start 69.85 67.2) (end 69.05 68) (width 0.25) (layer "F.Cu") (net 9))
 (segment (start 65.455 67.445) (end 65.455 66.975) (width 0.25) (layer "F.Cu") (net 9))
 (segment (start 64.825 65.575) (end 65.455 66.205) (width 0.25) (layer "F.Cu") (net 9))
 (segment (start 66.8 54.99) (end 67.14 54.65) (width 0.25) (layer "F.Cu") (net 9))
 (segment (start 70.741589 63.701589) (end 69.85 64.593178) (width 0.25) (layer "F.Cu") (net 9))
 (segment (start 61.925 65.435) (end 63.145 65.435) (width 0.25) (layer "F.Cu") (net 9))
 (segment (start 69.05 68) (end 66.01 68) (width 0.25) (layer "F.Cu") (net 9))
 (segment (start 69.85 64.593178) (end 69.85 67.2) (width 0.25) (layer "F.Cu") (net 9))
 (segment (start 64.77 65.43) (end 64.825 65.375) (width 0.25) (layer "F.Cu") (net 9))
 (via (at 70.741589 63.701589) (size 0.6) (drill 0.3) (layers "F.Cu" "B.Cu") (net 9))
 (via (at 66.8 54.99) (size 0.6) (drill 0.3) (layers "F.Cu" "B.Cu") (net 9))
 (segment (start 68.83 54.99) (end 66.8 54.99) (width 0.25) (layer "B.Cu") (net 9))
 (segment (start 71.65 57.81) (end 68.83 54.99) (width 0.25) (layer "B.Cu") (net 9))
 (segment (start 70.741589 63.701589) (end 71.65 62.793178) (width 0.25) (layer "B.Cu") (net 9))
 (segment (start 71.65 62.793178) (end 71.65 57.81) (width 0.25) (layer "B.Cu") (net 9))
 (segment (start 68.45 62.54) (end 68.87 62.54) (width 0.25) (layer "F.Cu") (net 1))
 (segment (start 67.1 62.81) (end 67.1 63.475) (width 0.25) (layer "F.Cu") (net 1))
 (segment (start 62.7 58.73) (end 63.02 58.73) (width 0.25) (layer "F.Cu") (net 1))
 (segment (start 63.02 58.73) (end 67.1 62.81) (width 0.25) (layer "F.Cu") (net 1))
 (segment (start 67.515 63.475) (end 68.45 62.54) (width 0.25) (layer "F.Cu") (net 1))
 (segment (start 67.1 63.475) (end 67.515 63.475) (width 0.25) (layer "F.Cu") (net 1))
 (segment (start 57.6 62.56) (end 58.89 61.27) (width 0.25) (layer "F.Cu") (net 2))
 (segment (start 57.6 63.225) (end 57.6 62.56) (width 0.25) (layer "F.Cu") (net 2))
 (segment (start 58.89 61.27) (end 62.7 61.27) (width 0.25) (layer "F.Cu") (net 2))
 (segment (start 64.825 63.475) (end 62.555 63.475) (width 0.25) (layer "F.Cu") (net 8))
 (segment (start 59.545 63.18) (end 59.5 63.225) (width 0.25) (layer "F.Cu") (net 8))
 (segment (start 62.26 63.18) (end 59.545 63.18) (width 0.25) (layer "F.Cu") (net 8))
 (segment (start 62.555 63.475) (end 62.26 63.18) (width 0.25) (layer "F.Cu") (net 8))
 (segment (start 67.1 66.84) (end 66.965 66.975) (width 0.25) (layer "F.Cu") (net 7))
 (segment (start 67.1 65.375) (end 67.1 66.69) (width 0.25) (layer "F.Cu") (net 7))
 (segment (start 67.1 66.69) (end 67.1 66.84) (width 0.25) (layer "F.Cu") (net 7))
 (segment (start 68.82 66.69) (end 68.88 66.63) (width 0.25) (layer "F.Cu") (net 7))
 (segment (start 66.965 66.975) (end 66.475 66.975) (width 0.25) (layer "F.Cu") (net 7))
 (segment (start 67.1 66.69) (end 68.82 66.69) (width 0.25) (layer "F.Cu") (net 7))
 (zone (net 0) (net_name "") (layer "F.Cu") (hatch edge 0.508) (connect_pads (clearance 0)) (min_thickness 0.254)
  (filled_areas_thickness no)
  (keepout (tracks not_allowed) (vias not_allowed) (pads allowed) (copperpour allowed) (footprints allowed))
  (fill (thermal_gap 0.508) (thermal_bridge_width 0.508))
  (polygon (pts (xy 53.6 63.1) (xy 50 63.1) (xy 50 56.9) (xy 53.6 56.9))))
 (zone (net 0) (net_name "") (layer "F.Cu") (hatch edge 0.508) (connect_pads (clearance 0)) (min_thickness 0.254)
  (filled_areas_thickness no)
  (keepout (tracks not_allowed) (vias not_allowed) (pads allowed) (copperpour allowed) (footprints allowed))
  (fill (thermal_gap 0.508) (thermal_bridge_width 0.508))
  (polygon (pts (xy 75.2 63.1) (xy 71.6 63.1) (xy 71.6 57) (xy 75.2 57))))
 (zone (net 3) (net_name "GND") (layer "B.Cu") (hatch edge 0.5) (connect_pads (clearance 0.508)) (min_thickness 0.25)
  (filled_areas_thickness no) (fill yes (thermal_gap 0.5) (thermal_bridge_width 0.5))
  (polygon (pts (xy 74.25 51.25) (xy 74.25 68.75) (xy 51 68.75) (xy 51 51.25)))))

